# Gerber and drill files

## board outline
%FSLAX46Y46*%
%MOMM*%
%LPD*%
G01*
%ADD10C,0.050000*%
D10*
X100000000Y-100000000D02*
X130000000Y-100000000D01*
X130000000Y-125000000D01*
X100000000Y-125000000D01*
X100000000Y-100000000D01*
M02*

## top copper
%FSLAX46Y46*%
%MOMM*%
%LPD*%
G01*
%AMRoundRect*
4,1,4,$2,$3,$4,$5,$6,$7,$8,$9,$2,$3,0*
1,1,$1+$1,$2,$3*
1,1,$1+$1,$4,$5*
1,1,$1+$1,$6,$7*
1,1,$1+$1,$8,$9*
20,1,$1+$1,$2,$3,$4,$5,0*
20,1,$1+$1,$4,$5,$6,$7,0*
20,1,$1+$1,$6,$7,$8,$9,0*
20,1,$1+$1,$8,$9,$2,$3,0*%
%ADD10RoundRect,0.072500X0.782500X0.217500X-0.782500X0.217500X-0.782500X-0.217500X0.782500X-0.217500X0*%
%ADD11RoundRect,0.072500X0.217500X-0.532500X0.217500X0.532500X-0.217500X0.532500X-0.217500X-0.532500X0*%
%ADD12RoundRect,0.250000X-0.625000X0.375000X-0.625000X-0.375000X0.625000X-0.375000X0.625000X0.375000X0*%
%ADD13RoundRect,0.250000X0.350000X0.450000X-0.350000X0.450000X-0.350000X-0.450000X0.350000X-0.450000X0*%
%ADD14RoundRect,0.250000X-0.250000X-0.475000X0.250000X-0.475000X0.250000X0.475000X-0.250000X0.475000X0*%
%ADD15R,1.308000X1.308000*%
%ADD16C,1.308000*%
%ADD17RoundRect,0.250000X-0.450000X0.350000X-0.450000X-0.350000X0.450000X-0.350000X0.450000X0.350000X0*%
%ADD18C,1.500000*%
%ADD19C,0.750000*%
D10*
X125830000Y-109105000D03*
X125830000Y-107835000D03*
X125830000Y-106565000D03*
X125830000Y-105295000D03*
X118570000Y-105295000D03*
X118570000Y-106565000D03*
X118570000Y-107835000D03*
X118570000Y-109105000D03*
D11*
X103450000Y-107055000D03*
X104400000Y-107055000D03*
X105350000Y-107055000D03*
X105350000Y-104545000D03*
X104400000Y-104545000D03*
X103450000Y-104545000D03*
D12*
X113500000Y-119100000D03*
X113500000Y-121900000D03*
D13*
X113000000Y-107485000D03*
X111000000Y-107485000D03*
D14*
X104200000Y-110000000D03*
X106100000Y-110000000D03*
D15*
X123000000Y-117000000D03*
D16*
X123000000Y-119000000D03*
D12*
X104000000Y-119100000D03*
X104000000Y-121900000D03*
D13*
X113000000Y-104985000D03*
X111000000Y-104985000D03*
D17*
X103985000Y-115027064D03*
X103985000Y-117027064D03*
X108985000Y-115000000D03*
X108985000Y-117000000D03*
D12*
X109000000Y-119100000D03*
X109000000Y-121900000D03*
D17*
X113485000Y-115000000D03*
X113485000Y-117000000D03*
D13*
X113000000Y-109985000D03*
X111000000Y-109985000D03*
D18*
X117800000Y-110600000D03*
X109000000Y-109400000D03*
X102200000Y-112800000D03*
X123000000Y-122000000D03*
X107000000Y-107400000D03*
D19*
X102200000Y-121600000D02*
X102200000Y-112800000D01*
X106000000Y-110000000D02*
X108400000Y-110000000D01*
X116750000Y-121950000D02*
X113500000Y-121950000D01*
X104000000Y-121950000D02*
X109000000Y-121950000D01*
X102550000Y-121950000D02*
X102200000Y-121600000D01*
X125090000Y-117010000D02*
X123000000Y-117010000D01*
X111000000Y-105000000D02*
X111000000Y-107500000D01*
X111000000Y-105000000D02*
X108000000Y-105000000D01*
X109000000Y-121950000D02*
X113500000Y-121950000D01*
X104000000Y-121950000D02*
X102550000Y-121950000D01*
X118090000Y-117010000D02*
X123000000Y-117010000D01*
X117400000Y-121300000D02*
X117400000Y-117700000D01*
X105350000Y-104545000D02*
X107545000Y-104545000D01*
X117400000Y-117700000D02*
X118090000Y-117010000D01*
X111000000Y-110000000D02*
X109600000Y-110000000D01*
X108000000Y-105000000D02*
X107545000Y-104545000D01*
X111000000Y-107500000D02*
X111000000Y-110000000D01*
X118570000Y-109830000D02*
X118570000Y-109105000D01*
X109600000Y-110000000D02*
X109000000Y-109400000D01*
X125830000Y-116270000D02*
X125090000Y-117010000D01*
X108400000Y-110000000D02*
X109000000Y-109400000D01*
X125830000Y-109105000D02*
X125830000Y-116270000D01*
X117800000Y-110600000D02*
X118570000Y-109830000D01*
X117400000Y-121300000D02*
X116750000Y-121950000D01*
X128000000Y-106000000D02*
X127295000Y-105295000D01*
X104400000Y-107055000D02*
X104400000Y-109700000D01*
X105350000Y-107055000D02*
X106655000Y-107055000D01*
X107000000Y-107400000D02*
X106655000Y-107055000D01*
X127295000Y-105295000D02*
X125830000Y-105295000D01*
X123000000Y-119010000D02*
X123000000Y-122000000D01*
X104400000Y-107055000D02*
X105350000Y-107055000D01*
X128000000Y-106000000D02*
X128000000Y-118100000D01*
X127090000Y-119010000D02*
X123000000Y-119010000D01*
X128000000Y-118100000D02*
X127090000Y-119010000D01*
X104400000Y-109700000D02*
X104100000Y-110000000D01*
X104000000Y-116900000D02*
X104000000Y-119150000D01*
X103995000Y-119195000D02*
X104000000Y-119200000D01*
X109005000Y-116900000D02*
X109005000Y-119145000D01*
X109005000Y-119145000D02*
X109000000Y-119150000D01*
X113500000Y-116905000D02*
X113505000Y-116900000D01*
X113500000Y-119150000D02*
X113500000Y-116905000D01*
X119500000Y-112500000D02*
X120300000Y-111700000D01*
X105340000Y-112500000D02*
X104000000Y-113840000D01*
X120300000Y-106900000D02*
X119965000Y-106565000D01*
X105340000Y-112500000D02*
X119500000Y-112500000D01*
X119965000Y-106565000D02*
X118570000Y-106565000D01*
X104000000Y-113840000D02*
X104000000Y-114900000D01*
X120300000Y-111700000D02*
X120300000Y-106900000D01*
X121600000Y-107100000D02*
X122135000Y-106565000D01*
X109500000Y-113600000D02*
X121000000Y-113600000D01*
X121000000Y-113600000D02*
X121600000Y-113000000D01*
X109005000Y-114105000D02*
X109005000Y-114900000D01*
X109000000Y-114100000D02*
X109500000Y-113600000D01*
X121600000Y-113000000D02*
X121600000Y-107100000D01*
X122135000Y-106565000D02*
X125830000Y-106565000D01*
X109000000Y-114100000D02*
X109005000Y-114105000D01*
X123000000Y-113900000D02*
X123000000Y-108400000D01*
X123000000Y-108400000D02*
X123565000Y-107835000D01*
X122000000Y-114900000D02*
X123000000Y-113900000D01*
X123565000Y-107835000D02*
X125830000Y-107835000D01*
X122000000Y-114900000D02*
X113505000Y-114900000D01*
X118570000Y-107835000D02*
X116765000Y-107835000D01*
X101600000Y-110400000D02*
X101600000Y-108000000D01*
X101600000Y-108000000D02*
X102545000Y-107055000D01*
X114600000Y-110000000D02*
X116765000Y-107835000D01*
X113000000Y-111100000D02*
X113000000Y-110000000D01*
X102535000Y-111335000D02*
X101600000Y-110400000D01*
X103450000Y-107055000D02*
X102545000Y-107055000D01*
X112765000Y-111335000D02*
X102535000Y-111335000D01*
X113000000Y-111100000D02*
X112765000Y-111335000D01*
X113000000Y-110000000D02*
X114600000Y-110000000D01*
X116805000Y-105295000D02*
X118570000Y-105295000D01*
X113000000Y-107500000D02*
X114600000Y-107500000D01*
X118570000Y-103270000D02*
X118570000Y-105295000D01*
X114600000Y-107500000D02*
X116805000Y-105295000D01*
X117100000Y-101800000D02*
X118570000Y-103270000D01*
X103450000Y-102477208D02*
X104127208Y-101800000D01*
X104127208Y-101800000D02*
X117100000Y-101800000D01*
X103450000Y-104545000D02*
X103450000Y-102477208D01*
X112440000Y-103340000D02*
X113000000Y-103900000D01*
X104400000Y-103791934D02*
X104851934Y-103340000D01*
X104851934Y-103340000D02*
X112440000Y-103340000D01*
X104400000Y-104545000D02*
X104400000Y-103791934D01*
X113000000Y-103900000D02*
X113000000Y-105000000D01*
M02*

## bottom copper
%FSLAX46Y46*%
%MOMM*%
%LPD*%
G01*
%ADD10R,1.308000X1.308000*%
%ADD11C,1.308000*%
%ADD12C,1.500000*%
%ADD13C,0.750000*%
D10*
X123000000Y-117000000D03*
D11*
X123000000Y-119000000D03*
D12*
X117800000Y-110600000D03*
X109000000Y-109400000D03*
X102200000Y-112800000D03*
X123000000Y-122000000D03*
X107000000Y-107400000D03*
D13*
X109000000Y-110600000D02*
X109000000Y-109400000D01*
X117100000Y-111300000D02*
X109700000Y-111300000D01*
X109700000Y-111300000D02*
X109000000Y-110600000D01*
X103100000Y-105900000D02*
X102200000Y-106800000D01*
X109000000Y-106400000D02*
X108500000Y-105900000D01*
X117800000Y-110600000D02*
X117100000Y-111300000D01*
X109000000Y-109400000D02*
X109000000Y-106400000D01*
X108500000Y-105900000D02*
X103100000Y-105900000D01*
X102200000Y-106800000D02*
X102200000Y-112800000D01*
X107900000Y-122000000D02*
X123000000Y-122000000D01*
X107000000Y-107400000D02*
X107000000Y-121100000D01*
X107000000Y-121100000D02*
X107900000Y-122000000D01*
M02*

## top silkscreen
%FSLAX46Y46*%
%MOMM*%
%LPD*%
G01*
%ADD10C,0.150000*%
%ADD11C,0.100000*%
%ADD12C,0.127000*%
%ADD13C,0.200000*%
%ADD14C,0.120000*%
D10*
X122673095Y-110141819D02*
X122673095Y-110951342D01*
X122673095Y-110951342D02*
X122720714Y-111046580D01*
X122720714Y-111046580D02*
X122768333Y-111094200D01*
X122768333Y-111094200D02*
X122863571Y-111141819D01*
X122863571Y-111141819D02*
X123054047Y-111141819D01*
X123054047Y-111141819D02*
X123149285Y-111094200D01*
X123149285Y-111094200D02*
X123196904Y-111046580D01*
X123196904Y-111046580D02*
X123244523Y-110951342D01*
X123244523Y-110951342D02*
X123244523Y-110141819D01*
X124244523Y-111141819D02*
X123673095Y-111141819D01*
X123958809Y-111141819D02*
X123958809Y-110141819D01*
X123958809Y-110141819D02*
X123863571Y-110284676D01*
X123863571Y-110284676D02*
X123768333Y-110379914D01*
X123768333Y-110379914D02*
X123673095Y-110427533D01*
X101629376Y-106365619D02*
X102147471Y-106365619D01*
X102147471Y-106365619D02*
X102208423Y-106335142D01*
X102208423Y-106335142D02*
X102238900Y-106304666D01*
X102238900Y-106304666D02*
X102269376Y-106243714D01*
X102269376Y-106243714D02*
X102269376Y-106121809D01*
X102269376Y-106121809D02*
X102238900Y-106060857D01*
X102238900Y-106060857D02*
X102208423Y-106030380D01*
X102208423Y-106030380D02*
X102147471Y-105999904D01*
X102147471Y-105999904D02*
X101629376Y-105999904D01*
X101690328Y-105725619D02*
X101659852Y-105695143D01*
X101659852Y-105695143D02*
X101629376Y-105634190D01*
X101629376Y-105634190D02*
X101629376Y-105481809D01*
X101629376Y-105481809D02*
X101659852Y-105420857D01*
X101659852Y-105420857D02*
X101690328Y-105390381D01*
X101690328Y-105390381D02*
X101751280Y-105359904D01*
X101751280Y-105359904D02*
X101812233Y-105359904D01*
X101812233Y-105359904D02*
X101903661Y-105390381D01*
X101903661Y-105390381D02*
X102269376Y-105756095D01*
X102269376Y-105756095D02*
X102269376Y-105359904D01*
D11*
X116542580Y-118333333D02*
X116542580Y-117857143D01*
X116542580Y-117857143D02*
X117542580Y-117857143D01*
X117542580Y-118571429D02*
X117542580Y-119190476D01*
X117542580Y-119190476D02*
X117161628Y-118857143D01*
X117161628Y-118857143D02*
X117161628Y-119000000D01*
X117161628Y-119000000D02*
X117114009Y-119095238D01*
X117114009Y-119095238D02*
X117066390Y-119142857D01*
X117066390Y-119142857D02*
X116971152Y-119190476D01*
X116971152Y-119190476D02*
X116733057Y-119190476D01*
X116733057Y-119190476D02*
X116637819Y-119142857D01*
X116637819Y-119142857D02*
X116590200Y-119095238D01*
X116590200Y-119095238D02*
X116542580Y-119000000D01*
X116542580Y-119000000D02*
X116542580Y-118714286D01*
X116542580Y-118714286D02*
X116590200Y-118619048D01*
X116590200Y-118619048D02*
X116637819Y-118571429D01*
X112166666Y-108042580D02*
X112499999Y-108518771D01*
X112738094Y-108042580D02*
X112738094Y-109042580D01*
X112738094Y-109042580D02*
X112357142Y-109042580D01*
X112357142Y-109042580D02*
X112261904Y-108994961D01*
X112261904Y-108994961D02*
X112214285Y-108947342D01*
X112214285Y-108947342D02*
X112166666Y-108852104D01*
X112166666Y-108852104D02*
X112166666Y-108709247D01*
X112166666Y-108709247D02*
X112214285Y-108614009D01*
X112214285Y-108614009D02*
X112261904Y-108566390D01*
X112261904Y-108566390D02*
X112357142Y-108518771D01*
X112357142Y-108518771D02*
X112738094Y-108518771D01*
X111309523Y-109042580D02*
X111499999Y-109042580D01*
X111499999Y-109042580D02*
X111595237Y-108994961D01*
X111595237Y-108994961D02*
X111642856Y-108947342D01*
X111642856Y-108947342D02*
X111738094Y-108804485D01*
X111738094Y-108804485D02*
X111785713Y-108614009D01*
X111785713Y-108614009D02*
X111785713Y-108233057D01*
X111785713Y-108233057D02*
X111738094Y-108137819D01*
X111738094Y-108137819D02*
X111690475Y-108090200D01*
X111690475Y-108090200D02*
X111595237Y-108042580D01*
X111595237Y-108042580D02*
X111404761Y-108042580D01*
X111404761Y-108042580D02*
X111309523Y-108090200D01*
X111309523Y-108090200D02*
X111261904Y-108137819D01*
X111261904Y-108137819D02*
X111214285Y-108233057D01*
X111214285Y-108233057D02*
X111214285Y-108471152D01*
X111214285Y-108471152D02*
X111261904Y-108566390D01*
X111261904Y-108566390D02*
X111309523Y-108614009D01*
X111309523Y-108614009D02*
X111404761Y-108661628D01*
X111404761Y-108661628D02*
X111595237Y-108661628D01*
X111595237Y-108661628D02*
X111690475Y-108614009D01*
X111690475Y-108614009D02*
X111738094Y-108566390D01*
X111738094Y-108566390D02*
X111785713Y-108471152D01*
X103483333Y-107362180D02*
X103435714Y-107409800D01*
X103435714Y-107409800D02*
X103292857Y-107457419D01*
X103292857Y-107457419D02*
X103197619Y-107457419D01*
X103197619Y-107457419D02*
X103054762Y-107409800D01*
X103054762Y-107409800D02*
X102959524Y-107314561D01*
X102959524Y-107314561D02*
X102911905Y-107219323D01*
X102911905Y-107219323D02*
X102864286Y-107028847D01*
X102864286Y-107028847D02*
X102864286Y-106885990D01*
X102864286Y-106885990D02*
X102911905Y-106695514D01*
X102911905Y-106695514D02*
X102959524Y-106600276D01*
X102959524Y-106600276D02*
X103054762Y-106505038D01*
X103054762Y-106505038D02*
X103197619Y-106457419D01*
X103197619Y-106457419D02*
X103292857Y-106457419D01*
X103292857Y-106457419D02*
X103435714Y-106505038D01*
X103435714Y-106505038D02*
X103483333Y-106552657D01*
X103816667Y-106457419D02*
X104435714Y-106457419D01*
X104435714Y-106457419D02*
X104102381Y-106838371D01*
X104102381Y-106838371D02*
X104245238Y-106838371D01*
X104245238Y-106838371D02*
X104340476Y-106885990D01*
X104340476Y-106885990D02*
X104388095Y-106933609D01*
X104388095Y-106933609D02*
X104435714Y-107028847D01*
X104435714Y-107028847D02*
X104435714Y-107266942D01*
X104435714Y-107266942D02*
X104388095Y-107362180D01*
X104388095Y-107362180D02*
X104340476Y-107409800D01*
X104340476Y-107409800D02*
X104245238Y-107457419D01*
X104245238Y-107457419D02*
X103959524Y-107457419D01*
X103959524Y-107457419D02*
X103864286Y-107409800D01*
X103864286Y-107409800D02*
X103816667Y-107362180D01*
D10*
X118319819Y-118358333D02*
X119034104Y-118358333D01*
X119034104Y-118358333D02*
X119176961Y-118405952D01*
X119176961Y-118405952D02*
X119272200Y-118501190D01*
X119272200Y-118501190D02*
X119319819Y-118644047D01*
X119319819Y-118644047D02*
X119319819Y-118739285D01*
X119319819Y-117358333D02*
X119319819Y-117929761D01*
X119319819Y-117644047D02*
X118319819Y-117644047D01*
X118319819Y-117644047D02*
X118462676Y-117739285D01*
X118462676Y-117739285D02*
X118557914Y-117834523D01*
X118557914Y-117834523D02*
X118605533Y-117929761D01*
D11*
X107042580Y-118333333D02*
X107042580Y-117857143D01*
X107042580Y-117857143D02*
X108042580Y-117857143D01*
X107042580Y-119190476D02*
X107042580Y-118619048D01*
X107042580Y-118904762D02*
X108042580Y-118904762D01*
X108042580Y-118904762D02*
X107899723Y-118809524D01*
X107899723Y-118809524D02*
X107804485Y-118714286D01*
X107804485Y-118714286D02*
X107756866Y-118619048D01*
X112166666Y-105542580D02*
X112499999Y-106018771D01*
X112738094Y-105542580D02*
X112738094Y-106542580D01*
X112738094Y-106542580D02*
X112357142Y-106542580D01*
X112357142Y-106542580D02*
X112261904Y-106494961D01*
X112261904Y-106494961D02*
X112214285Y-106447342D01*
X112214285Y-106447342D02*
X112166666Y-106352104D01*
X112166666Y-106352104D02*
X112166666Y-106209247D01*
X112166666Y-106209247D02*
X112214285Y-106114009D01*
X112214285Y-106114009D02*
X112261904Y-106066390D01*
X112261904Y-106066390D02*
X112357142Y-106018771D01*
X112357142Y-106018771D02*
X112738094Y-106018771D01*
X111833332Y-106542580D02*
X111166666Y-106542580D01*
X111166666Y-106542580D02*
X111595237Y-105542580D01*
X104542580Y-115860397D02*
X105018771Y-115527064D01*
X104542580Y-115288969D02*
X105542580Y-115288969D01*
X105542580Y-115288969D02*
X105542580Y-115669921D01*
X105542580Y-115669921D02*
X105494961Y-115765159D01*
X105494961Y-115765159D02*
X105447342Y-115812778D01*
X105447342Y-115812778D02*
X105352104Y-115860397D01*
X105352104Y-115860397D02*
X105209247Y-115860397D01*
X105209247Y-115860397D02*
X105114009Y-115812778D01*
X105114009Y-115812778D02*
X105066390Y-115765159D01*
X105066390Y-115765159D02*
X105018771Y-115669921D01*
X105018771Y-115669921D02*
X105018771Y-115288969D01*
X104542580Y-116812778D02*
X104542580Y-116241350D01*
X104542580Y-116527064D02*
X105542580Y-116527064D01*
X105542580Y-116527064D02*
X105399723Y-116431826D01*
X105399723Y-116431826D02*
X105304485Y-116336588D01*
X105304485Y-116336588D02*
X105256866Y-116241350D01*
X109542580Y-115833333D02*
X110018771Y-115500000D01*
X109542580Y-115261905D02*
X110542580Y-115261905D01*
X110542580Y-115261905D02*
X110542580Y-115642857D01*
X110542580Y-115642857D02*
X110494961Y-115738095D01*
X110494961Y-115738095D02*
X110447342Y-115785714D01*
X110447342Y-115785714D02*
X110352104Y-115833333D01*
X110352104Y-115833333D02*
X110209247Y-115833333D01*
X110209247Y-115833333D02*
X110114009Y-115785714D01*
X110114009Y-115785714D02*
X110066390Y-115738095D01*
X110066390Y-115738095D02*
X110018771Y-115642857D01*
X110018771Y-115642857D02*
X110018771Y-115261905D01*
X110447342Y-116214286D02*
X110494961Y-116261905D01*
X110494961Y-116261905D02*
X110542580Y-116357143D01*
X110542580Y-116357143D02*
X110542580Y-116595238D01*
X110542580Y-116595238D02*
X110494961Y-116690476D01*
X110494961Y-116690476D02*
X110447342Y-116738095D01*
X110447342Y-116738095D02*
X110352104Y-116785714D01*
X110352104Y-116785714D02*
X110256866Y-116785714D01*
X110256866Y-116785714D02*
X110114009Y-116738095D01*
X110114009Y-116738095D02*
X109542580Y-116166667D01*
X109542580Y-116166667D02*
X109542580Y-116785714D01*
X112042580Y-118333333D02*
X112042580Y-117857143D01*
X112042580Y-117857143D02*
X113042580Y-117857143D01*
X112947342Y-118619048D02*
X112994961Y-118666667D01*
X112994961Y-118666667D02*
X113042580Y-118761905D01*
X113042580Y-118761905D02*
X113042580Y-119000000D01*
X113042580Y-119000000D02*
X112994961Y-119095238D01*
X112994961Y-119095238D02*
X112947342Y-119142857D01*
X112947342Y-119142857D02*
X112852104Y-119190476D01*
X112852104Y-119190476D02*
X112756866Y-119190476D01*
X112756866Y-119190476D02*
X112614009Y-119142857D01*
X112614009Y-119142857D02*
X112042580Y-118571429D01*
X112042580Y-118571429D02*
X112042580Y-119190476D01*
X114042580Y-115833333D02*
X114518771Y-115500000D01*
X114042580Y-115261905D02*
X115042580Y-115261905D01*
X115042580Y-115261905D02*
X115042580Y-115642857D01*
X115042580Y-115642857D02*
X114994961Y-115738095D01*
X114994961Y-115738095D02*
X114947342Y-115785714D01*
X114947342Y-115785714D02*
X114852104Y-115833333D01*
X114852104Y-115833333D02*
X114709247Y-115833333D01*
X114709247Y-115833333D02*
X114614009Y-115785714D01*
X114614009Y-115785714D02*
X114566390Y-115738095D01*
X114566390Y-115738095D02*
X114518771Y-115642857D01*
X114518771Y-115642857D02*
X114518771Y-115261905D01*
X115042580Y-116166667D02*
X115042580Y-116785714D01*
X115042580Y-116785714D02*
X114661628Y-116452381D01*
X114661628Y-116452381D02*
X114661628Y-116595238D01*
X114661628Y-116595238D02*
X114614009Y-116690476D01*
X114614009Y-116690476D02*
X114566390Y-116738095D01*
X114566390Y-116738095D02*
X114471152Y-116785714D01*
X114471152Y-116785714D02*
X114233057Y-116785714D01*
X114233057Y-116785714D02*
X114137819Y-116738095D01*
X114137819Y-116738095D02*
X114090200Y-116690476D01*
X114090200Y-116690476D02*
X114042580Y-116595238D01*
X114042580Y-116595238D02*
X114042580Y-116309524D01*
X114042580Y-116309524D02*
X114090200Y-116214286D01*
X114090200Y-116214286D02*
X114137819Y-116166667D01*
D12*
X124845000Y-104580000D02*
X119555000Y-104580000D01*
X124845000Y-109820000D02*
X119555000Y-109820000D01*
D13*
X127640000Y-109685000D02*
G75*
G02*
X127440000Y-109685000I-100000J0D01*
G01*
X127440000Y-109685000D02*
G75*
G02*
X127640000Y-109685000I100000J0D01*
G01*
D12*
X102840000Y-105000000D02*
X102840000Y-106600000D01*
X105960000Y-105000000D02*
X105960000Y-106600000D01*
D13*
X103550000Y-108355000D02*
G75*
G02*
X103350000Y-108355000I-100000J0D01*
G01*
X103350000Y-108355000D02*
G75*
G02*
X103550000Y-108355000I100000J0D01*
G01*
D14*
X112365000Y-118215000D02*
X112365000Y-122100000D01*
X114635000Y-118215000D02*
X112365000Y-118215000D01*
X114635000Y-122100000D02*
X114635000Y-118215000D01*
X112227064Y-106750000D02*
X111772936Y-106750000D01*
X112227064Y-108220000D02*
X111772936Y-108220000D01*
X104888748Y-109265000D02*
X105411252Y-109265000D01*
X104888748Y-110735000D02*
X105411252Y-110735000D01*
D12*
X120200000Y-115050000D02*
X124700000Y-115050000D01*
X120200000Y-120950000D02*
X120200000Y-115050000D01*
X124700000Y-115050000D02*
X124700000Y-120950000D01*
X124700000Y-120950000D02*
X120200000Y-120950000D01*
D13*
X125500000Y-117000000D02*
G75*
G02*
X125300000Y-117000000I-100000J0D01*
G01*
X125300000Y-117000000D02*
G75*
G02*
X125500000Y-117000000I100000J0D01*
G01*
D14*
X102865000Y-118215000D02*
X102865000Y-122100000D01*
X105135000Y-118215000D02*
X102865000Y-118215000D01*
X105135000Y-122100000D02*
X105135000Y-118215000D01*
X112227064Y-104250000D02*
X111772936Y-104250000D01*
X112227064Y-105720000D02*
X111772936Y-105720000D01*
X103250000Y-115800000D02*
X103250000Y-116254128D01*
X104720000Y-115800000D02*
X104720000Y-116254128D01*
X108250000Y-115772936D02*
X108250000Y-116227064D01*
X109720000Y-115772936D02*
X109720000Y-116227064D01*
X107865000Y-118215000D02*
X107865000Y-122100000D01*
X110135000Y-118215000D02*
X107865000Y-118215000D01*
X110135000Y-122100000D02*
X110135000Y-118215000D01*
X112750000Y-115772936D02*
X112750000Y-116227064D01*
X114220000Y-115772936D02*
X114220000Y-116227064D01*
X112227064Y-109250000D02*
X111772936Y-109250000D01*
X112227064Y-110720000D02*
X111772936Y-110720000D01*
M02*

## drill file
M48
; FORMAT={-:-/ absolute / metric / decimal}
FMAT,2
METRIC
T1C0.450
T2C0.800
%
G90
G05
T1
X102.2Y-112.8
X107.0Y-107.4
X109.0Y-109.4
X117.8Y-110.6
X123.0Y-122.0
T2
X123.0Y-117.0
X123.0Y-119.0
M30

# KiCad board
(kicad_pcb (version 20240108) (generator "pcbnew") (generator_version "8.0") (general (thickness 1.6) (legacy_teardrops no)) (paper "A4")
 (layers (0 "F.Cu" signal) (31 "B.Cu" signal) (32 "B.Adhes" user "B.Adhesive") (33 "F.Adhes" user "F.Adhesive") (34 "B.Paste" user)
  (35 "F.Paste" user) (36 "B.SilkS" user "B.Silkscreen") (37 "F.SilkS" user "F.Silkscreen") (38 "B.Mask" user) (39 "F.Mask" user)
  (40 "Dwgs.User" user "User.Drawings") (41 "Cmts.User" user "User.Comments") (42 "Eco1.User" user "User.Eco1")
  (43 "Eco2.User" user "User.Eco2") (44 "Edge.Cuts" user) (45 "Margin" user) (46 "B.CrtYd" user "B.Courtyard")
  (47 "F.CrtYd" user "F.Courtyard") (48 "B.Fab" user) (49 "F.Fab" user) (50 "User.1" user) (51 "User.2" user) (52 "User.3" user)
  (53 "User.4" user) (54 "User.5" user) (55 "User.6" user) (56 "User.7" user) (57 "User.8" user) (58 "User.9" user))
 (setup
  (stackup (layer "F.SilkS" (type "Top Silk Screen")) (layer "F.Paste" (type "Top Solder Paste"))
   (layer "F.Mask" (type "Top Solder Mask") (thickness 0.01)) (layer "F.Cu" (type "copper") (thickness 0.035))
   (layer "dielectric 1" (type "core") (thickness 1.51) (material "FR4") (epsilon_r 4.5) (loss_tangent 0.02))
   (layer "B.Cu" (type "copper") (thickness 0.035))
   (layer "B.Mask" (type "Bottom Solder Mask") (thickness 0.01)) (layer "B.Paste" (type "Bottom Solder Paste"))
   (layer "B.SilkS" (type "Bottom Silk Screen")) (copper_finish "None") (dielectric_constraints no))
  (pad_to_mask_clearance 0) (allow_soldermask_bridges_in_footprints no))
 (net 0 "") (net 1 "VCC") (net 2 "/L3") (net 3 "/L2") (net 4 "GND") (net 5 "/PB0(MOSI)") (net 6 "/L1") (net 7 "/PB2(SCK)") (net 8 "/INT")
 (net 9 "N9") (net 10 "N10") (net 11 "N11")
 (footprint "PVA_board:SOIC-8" (layer "F.Cu") (at 122.2 107.2 180)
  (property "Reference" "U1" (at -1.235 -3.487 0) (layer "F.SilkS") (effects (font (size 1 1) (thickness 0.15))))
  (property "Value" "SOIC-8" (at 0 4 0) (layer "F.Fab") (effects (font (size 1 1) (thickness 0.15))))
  (fp_line (start -2.645 2.62) (end 2.645 2.62) (stroke (width 0.127) (type solid)) (layer "F.SilkS"))
  (fp_line (start -2.645 -2.62) (end 2.645 -2.62) (stroke (width 0.127) (type solid)) (layer "F.SilkS"))
  (fp_circle (center -5.34 -2.485) (end -5.24 -2.485) (stroke (width 0.2) (type solid)) (fill none) (layer "F.SilkS"))
  (pad "1" smd roundrect (at -3.63 -1.905 180) (size 1.71 0.58) (layers "F.Cu" "F.Paste" "F.Mask") (roundrect_rratio 0.125) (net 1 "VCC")
   (solder_mask_margin 0.102))
  (pad "2" smd roundrect (at -3.63 -0.635 180) (size 1.71 0.58) (layers "F.Cu" "F.Paste" "F.Mask") (roundrect_rratio 0.125) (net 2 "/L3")
   (solder_mask_margin 0.102))
  (pad "3" smd roundrect (at -3.63 0.635 180) (size 1.71 0.58) (layers "F.Cu" "F.Paste" "F.Mask") (roundrect_rratio 0.125) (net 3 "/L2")
   (solder_mask_margin 0.102))
  (pad "4" smd roundrect (at -3.63 1.905 180) (size 1.71 0.58) (layers "F.Cu" "F.Paste" "F.Mask") (roundrect_rratio 0.125) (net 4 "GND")
   (solder_mask_margin 0.102))
  (pad "5" smd roundrect (at 3.63 1.905 180) (size 1.71 0.58) (layers "F.Cu" "F.Paste" "F.Mask") (roundrect_rratio 0.125)
   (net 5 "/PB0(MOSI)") (solder_mask_margin 0.102))
  (pad "6" smd roundrect (at 3.63 0.635 180) (size 1.71 0.58) (layers "F.Cu" "F.Paste" "F.Mask") (roundrect_rratio 0.125) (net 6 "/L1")
   (solder_mask_margin 0.102))
  (pad "7" smd roundrect (at 3.63 -0.635 180) (size 1.71 0.58) (layers "F.Cu" "F.Paste" "F.Mask") (roundrect_rratio 0.125)
   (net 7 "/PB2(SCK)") (solder_mask_margin 0.102))
  (pad "8" smd roundrect (at 3.63 -1.905 180) (size 1.71 0.58) (layers "F.Cu" "F.Paste" "F.Mask") (roundrect_rratio 0.125) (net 1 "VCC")
   (solder_mask_margin 0.102)))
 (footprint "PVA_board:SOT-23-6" (layer "F.Cu") (at 104.4 105.8 90)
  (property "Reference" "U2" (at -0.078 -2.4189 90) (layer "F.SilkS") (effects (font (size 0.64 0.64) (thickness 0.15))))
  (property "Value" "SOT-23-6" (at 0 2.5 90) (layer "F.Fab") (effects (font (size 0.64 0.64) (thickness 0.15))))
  (fp_line (start 0.8 -1.56) (end -0.8 -1.56) (stroke (width 0.127) (type solid)) (layer "F.SilkS"))
  (fp_line (start 0.8 1.56) (end -0.8 1.56) (stroke (width 0.127) (type solid)) (layer "F.SilkS"))
  (fp_circle (center -2.555 -0.95) (end -2.455 -0.95) (stroke (width 0.2) (type solid)) (fill none) (layer "F.SilkS"))
  (pad "1" smd roundrect (at -1.255 -0.95 90) (size 1.21 0.58) (layers "F.Cu" "F.Paste" "F.Mask") (roundrect_rratio 0.125)
   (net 7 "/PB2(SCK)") (solder_mask_margin 0.102))
  (pad "2" smd roundrect (at -1.255 0 90) (size 1.21 0.58) (layers "F.Cu" "F.Paste" "F.Mask") (roundrect_rratio 0.125) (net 4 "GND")
   (solder_mask_margin 0.102))
  (pad "3" smd roundrect (at -1.255 0.95 90) (size 1.21 0.58) (layers "F.Cu" "F.Paste" "F.Mask") (roundrect_rratio 0.125) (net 4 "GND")
   (solder_mask_margin 0.102))
  (pad "4" smd roundrect (at 1.255 0.95 90) (size 1.21 0.58) (layers "F.Cu" "F.Paste" "F.Mask") (roundrect_rratio 0.125) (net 1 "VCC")
   (solder_mask_margin 0.102))
  (pad "5" smd roundrect (at 1.255 0 90) (size 1.21 0.58) (layers "F.Cu" "F.Paste" "F.Mask") (roundrect_rratio 0.125) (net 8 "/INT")
   (solder_mask_margin 0.102))
  (pad "6" smd roundrect (at 1.255 -0.95 90) (size 1.21 0.58) (layers "F.Cu" "F.Paste" "F.Mask") (roundrect_rratio 0.125)
   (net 5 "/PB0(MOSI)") (solder_mask_margin 0.102)))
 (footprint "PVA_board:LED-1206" (layer "F.Cu") (at 113.5 120.5 -90)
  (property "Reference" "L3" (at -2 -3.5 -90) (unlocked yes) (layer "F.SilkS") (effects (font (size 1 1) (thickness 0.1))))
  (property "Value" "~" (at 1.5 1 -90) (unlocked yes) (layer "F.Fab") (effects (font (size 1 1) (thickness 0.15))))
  (fp_line (start -2.285 1.135) (end 1.6 1.135) (stroke (width 0.12) (type solid)) (layer "F.SilkS"))
  (fp_line (start -2.285 -1.135) (end -2.285 1.135) (stroke (width 0.12) (type solid)) (layer "F.SilkS"))
  (fp_line (start 1.6 -1.135) (end -2.285 -1.135) (stroke (width 0.12) (type solid)) (layer "F.SilkS"))
  (pad "1" smd roundrect (at -1.4 0 270) (size 1.25 1.75) (layers "F.Cu" "F.Paste" "F.Mask") (roundrect_rratio 0.2) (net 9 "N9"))
  (pad "2" smd roundrect (at 1.4 0 270) (size 1.25 1.75) (layers "F.Cu" "F.Paste" "F.Mask") (roundrect_rratio 0.2) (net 1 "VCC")))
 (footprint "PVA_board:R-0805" (layer "F.Cu") (at 112 107.5 180)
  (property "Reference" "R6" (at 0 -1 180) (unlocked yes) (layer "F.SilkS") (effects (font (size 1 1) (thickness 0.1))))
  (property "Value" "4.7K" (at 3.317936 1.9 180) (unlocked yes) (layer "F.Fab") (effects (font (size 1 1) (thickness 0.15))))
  (fp_line (start -0.227064 0.75) (end 0.227064 0.75) (stroke (width 0.12) (type solid)) (layer "F.SilkS"))
  (fp_line (start -0.227064 -0.72) (end 0.227064 -0.72) (stroke (width 0.12) (type solid)) (layer "F.SilkS"))
  (pad "1" smd roundrect (at -1 0.015 180) (size 1.2 1.4) (layers "F.Cu" "F.Paste" "F.Mask") (roundrect_rratio 0.208333)
   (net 5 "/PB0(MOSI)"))
  (pad "2" smd roundrect (at 1 0.015 180) (size 1.2 1.4) (layers "F.Cu" "F.Paste" "F.Mask") (roundrect_rratio 0.208333) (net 1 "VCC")))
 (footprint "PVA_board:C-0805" (layer "F.Cu") (at 105.15 110)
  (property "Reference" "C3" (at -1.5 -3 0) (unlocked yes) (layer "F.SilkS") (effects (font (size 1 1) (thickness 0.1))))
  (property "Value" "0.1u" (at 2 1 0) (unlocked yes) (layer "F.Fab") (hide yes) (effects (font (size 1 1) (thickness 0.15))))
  (fp_line (start -0.261252 -0.735) (end 0.261252 -0.735) (stroke (width 0.12) (type solid)) (layer "F.SilkS"))
  (fp_line (start -0.261252 0.735) (end 0.261252 0.735) (stroke (width 0.12) (type solid)) (layer "F.SilkS"))
  (pad "1" smd roundrect (at -0.95 0) (size 1 1.45) (layers "F.Cu" "F.Paste" "F.Mask") (roundrect_rratio 0.25) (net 4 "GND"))
  (pad "2" smd roundrect (at 0.95 0) (size 1 1.45) (layers "F.Cu" "F.Paste" "F.Mask") (roundrect_rratio 0.25) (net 1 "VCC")))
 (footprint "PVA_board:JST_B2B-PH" (layer "F.Cu") (at 123 118 90)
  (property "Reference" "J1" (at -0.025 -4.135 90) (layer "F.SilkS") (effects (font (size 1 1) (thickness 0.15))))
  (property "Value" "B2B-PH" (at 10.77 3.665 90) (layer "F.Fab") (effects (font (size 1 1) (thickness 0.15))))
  (fp_line (start 2.95 -2.8) (end 2.95 1.7) (stroke (width 0.127) (type solid)) (layer "F.SilkS"))
  (fp_line (start -2.95 -2.8) (end 2.95 -2.8) (stroke (width 0.127) (type solid)) (layer "F.SilkS"))
  (fp_line (start 2.95 1.7) (end -2.95 1.7) (stroke (width 0.127) (type solid)) (layer "F.SilkS"))
  (fp_line (start -2.95 1.7) (end -2.95 -2.8) (stroke (width 0.127) (type solid)) (layer "F.SilkS"))
  (fp_circle (center 1 2.4) (end 1.1 2.4) (stroke (width 0.2) (type solid)) (fill none) (layer "F.SilkS"))
  (pad "1" thru_hole rect (at 1 0 90) (size 1.308 1.308) (drill 0.8) (layers "*.Cu" "*.Mask") (remove_unused_layers no) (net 1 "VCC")
   (solder_mask_margin 0.102))
  (pad "2" thru_hole circle (at -1 0 90) (size 1.308 1.308) (drill 0.8) (layers "*.Cu" "*.Mask") (remove_unused_layers no) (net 4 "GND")
   (solder_mask_margin 0.102)))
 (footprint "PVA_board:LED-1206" (layer "F.Cu") (at 104 120.5 -90)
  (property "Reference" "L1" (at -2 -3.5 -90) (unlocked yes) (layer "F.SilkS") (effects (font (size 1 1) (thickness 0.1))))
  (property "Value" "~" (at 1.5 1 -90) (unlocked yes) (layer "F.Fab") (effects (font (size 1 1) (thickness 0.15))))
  (fp_line (start -2.285 1.135) (end 1.6 1.135) (stroke (width 0.12) (type solid)) (layer "F.SilkS"))
  (fp_line (start -2.285 -1.135) (end -2.285 1.135) (stroke (width 0.12) (type solid)) (layer "F.SilkS"))
  (fp_line (start 1.6 -1.135) (end -2.285 -1.135) (stroke (width 0.12) (type solid)) (layer "F.SilkS"))
  (pad "1" smd roundrect (at -1.4 0 270) (size 1.25 1.75) (layers "F.Cu" "F.Paste" "F.Mask") (roundrect_rratio 0.2) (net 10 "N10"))
  (pad "2" smd roundrect (at 1.4 0 270) (size 1.25 1.75) (layers "F.Cu" "F.Paste" "F.Mask") (roundrect_rratio 0.2) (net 1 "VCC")))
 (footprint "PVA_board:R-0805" (layer "F.Cu") (at 112 105 180)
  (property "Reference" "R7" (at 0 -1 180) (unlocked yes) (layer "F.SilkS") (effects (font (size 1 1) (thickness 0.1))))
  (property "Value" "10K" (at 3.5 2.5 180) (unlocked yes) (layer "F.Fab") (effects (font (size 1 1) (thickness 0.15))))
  (fp_line (start -0.227064 0.75) (end 0.227064 0.75) (stroke (width 0.12) (type solid)) (layer "F.SilkS"))
  (fp_line (start -0.227064 -0.72) (end 0.227064 -0.72) (stroke (width 0.12) (type solid)) (layer "F.SilkS"))
  (pad "1" smd roundrect (at -1 0.015 180) (size 1.2 1.4) (layers "F.Cu" "F.Paste" "F.Mask") (roundrect_rratio 0.208333) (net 8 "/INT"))
  (pad "2" smd roundrect (at 1 0.015 180) (size 1.2 1.4) (layers "F.Cu" "F.Paste" "F.Mask") (roundrect_rratio 0.208333) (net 1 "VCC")))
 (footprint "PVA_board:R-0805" (layer "F.Cu") (at 104 116.027064 -90)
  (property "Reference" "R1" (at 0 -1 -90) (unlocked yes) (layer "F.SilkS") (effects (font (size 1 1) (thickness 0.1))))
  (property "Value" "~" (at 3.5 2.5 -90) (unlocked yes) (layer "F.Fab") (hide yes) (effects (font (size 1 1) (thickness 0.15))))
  (fp_line (start -0.227064 0.75) (end 0.227064 0.75) (stroke (width 0.12) (type solid)) (layer "F.SilkS"))
  (fp_line (start -0.227064 -0.72) (end 0.227064 -0.72) (stroke (width 0.12) (type solid)) (layer "F.SilkS"))
  (pad "1" smd roundrect (at -1 0.015 270) (size 1.2 1.4) (layers "F.Cu" "F.Paste" "F.Mask") (roundrect_rratio 0.208333) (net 6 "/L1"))
  (pad "2" smd roundrect (at 1 0.015 270) (size 1.2 1.4) (layers "F.Cu" "F.Paste" "F.Mask") (roundrect_rratio 0.208333) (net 10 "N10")))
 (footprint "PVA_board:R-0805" (layer "F.Cu") (at 109 116 -90)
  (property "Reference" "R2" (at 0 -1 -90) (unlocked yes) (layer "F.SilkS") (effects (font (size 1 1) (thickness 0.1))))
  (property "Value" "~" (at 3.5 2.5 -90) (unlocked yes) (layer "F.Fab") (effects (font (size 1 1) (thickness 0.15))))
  (fp_line (start -0.227064 0.75) (end 0.227064 0.75) (stroke (width 0.12) (type solid)) (layer "F.SilkS"))
  (fp_line (start -0.227064 -0.72) (end 0.227064 -0.72) (stroke (width 0.12) (type solid)) (layer "F.SilkS"))
  (pad "1" smd roundrect (at -1 0.015 270) (size 1.2 1.4) (layers "F.Cu" "F.Paste" "F.Mask") (roundrect_rratio 0.208333) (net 3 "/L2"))
  (pad "2" smd roundrect (at 1 0.015 270) (size 1.2 1.4) (layers "F.Cu" "F.Paste" "F.Mask") (roundrect_rratio 0.208333) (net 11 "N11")))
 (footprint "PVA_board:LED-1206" (layer "F.Cu") (at 109 120.5 -90)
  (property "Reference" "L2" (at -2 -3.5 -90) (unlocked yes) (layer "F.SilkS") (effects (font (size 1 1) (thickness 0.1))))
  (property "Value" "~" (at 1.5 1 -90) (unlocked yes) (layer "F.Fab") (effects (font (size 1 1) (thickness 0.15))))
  (fp_line (start -2.285 1.135) (end 1.6 1.135) (stroke (width 0.12) (type solid)) (layer "F.SilkS"))
  (fp_line (start -2.285 -1.135) (end -2.285 1.135) (stroke (width 0.12) (type solid)) (layer "F.SilkS"))
  (fp_line (start 1.6 -1.135) (end -2.285 -1.135) (stroke (width 0.12) (type solid)) (layer "F.SilkS"))
  (pad "1" smd roundrect (at -1.4 0 270) (size 1.25 1.75) (layers "F.Cu" "F.Paste" "F.Mask") (roundrect_rratio 0.2) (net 11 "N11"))
  (pad "2" smd roundrect (at 1.4 0 270) (size 1.25 1.75) (layers "F.Cu" "F.Paste" "F.Mask") (roundrect_rratio 0.2) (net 1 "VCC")))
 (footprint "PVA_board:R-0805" (layer "F.Cu") (at 113.5 116 -90)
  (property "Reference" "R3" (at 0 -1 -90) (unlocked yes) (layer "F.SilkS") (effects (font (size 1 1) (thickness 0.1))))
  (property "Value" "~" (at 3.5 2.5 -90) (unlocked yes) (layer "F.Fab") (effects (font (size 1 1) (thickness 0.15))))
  (fp_line (start -0.227064 0.75) (end 0.227064 0.75) (stroke (width 0.12) (type solid)) (layer "F.SilkS"))
  (fp_line (start -0.227064 -0.72) (end 0.227064 -0.72) (stroke (width 0.12) (type solid)) (layer "F.SilkS"))
  (pad "1" smd roundrect (at -1 0.015 270) (size 1.2 1.4) (layers "F.Cu" "F.Paste" "F.Mask") (roundrect_rratio 0.208333) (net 2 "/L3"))
  (pad "2" smd roundrect (at 1 0.015 270) (size 1.2 1.4) (layers "F.Cu" "F.Paste" "F.Mask") (roundrect_rratio 0.208333) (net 9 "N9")))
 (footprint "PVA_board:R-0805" (layer "F.Cu") (at 112 110 180)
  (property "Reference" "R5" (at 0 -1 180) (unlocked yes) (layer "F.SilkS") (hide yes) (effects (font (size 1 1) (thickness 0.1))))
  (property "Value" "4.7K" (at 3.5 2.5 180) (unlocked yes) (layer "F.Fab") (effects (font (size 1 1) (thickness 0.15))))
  (fp_line (start -0.227064 0.75) (end 0.227064 0.75) (stroke (width 0.12) (type solid)) (layer "F.SilkS"))
  (fp_line (start -0.227064 -0.72) (end 0.227064 -0.72) (stroke (width 0.12) (type solid)) (layer "F.SilkS"))
  (pad "1" smd roundrect (at -1 0.015 180) (size 1.2 1.4) (layers "F.Cu" "F.Paste" "F.Mask") (roundrect_rratio 0.208333) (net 7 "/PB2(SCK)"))
  (pad "2" smd roundrect (at 1 0.015 180) (size 1.2 1.4) (layers "F.Cu" "F.Paste" "F.Mask") (roundrect_rratio 0.208333) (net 1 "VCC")))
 (gr_rect (start 100 100) (end 130 125) (stroke (width 0.05) (type default)) (fill none) (layer "Edge.Cuts"))
 (segment (start 102.2 121.6) (end 102.2 112.8) (width 0.75) (layer "F.Cu") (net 1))
 (segment (start 106 110) (end 108.4 110) (width 0.75) (layer "F.Cu") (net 1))
 (segment (start 116.75 121.95) (end 113.5 121.95) (width 0.75) (layer "F.Cu") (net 1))
 (segment (start 104 121.95) (end 109 121.95) (width 0.75) (layer "F.Cu") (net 1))
 (segment (start 102.55 121.95) (end 102.2 121.6) (width 0.75) (layer "F.Cu") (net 1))
 (segment (start 125.09 117.01) (end 123 117.01) (width 0.75) (layer "F.Cu") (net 1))
 (segment (start 111 105) (end 111 107.5) (width 0.75) (layer "F.Cu") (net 1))
 (segment (start 111 105) (end 108 105) (width 0.75) (layer "F.Cu") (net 1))
 (segment (start 109 121.95) (end 113.5 121.95) (width 0.75) (layer "F.Cu") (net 1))
 (segment (start 104 121.95) (end 102.55 121.95) (width 0.75) (layer "F.Cu") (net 1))
 (segment (start 118.09 117.01) (end 123 117.01) (width 0.75) (layer "F.Cu") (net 1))
 (segment (start 117.4 121.3) (end 117.4 117.7) (width 0.75) (layer "F.Cu") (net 1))
 (segment (start 105.35 104.545) (end 107.545 104.545) (width 0.75) (layer "F.Cu") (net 1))
 (segment (start 117.4 117.7) (end 118.09 117.01) (width 0.75) (layer "F.Cu") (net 1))
 (segment (start 111 110) (end 109.6 110) (width 0.75) (layer "F.Cu") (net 1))
 (segment (start 108 105) (end 107.545 104.545) (width 0.75) (layer "F.Cu") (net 1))
 (segment (start 111 107.5) (end 111 110) (width 0.75) (layer "F.Cu") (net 1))
 (segment (start 118.57 109.83) (end 118.57 109.105) (width 0.75) (layer "F.Cu") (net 1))
 (segment (start 109.6 110) (end 109 109.4) (width 0.75) (layer "F.Cu") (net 1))
 (segment (start 125.83 116.27) (end 125.09 117.01) (width 0.75) (layer "F.Cu") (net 1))
 (segment (start 108.4 110) (end 109 109.4) (width 0.75) (layer "F.Cu") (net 1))
 (segment (start 125.83 109.105) (end 125.83 116.27) (width 0.75) (layer "F.Cu") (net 1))
 (segment (start 117.8 110.6) (end 118.57 109.83) (width 0.75) (layer "F.Cu") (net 1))
 (segment (start 117.4 121.3) (end 116.75 121.95) (width 0.75) (layer "F.Cu") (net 1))
 (via (at 117.8 110.6) (size 1.5) (drill 0.45) (layers "F.Cu" "B.Cu") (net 1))
 (via (at 109 109.4) (size 1.5) (drill 0.45) (layers "F.Cu" "B.Cu") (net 1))
 (via (at 102.2 112.8) (size 1.5) (drill 0.45) (layers "F.Cu" "B.Cu") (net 1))
 (segment (start 109 110.6) (end 109 109.4) (width 0.75) (layer "B.Cu") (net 1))
 (segment (start 117.1 111.3) (end 109.7 111.3) (width 0.75) (layer "B.Cu") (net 1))
 (segment (start 109.7 111.3) (end 109 110.6) (width 0.75) (layer "B.Cu") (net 1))
 (segment (start 103.1 105.9) (end 102.2 106.8) (width 0.75) (layer "B.Cu") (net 1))
 (segment (start 109 106.4) (end 108.5 105.9) (width 0.75) (layer "B.Cu") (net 1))
 (segment (start 117.8 110.6) (end 117.1 111.3) (width 0.75) (layer "B.Cu") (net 1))
 (segment (start 109 109.4) (end 109 106.4) (width 0.75) (layer "B.Cu") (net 1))
 (segment (start 108.5 105.9) (end 103.1 105.9) (width 0.75) (layer "B.Cu") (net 1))
 (segment (start 102.2 106.8) (end 102.2 112.8) (width 0.75) (layer "B.Cu") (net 1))
 (segment (start 128 106) (end 127.295 105.295) (width 0.75) (layer "F.Cu") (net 4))
 (segment (start 104.4 107.055) (end 104.4 109.7) (width 0.75) (layer "F.Cu") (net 4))
 (segment (start 105.35 107.055) (end 106.655 107.055) (width 0.75) (layer "F.Cu") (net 4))
 (segment (start 107 107.4) (end 106.655 107.055) (width 0.75) (layer "F.Cu") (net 4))
 (segment (start 127.295 105.295) (end 125.83 105.295) (width 0.75) (layer "F.Cu") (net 4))
 (segment (start 123 119.01) (end 123 122) (width 0.75) (layer "F.Cu") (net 4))
 (segment (start 104.4 107.055) (end 105.35 107.055) (width 0.75) (layer "F.Cu") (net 4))
 (segment (start 128 106) (end 128 118.1) (width 0.75) (layer "F.Cu") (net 4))
 (segment (start 127.09 119.01) (end 123 119.01) (width 0.75) (layer "F.Cu") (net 4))
 (segment (start 128 118.1) (end 127.09 119.01) (width 0.75) (layer "F.Cu") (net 4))
 (segment (start 104.4 109.7) (end 104.1 110) (width 0.75) (layer "F.Cu") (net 4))
 (via (at 123 122) (size 1.5) (drill 0.45) (layers "F.Cu" "B.Cu") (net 4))
 (via (at 107 107.4) (size 1.5) (drill 0.45) (layers "F.Cu" "B.Cu") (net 4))
 (segment (start 107.9 122) (end 123 122) (width 0.75) (layer "B.Cu") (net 4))
 (segment (start 107 107.4) (end 107 121.1) (width 0.75) (layer "B.Cu") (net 4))
 (segment (start 107 121.1) (end 107.9 122) (width 0.75) (layer "B.Cu") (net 4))
 (segment (start 104 116.9) (end 104 119.15) (width 0.75) (layer "F.Cu") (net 10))
 (segment (start 103.995 119.195) (end 104 119.2) (width 0.75) (layer "F.Cu") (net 10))
 (segment (start 109.005 116.9) (end 109.005 119.145) (width 0.75) (layer "F.Cu") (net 11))
 (segment (start 109.005 119.145) (end 109 119.15) (width 0.75) (layer "F.Cu") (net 11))
 (segment (start 113.5 116.905) (end 113.505 116.9) (width 0.75) (layer "F.Cu") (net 9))
 (segment (start 113.5 119.15) (end 113.5 116.905) (width 0.75) (layer "F.Cu") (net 9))
 (segment (start 119.5 112.5) (end 120.3 111.7) (width 0.75) (layer "F.Cu") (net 6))
 (segment (start 105.34 112.5) (end 104 113.84) (width 0.75) (layer "F.Cu") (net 6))
 (segment (start 120.3 106.9) (end 119.965 106.565) (width 0.75) (layer "F.Cu") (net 6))
 (segment (start 105.34 112.5) (end 119.5 112.5) (width 0.75) (layer "F.Cu") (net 6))
 (segment (start 119.965 106.565) (end 118.57 106.565) (width 0.75) (layer "F.Cu") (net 6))
 (segment (start 104 113.84) (end 104 114.9) (width 0.75) (layer "F.Cu") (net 6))
 (segment (start 120.3 111.7) (end 120.3 106.9) (width 0.75) (layer "F.Cu") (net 6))
 (segment (start 121.6 107.1) (end 122.135 106.565) (width 0.75) (layer "F.Cu") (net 3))
 (segment (start 109.5 113.6) (end 121 113.6) (width 0.75) (layer "F.Cu") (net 3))
 (segment (start 121 113.6) (end 121.6 113) (width 0.75) (layer "F.Cu") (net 3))
 (segment (start 109.005 114.105) (end 109.005 114.9) (width 0.75) (layer "F.Cu") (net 3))
 (segment (start 109 114.1) (end 109.5 113.6) (width 0.75) (layer "F.Cu") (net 3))
 (segment (start 121.6 113) (end 121.6 107.1) (width 0.75) (layer "F.Cu") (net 3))
 (segment (start 122.135 106.565) (end 125.83 106.565) (width 0.75) (layer "F.Cu") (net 3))
 (segment (start 109 114.1) (end 109.005 114.105) (width 0.75) (layer "F.Cu") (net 3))
 (segment (start 123 113.9) (end 123 108.4) (width 0.75) (layer "F.Cu") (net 2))
 (segment (start 123 108.4) (end 123.565 107.835) (width 0.75) (layer "F.Cu") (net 2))
 (segment (start 122 114.9) (end 123 113.9) (width 0.75) (layer "F.Cu") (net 2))
 (segment (start 123.565 107.835) (end 125.83 107.835) (width 0.75) (layer "F.Cu") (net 2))
 (segment (start 122 114.9) (end 113.505 114.9) (width 0.75) (layer "F.Cu") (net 2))
 (segment (start 118.57 107.835) (end 116.765 107.835) (width 0.75) (layer "F.Cu") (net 7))
 (segment (start 101.6 110.4) (end 101.6 108) (width 0.75) (layer "F.Cu") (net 7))
 (segment (start 101.6 108) (end 102.545 107.055) (width 0.75) (layer "F.Cu") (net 7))
 (segment (start 114.6 110) (end 116.765 107.835) (width 0.75) (layer "F.Cu") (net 7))
 (segment (start 113 111.1) (end 113 110) (width 0.75) (layer "F.Cu") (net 7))
 (segment (start 102.535 111.335) (end 101.6 110.4) (width 0.75) (layer "F.Cu") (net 7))
 (segment (start 103.45 107.055) (end 102.545 107.055) (width 0.75) (layer "F.Cu") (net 7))
 (segment (start 112.765 111.335) (end 102.535 111.335) (width 0.75) (layer "F.Cu") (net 7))
 (segment (start 113 111.1) (end 112.765 111.335) (width 0.75) (layer "F.Cu") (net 7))
 (segment (start 113 110) (end 114.6 110) (width 0.75) (layer "F.Cu") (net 7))
 (segment (start 116.805 105.295) (end 118.57 105.295) (width 0.75) (layer "F.Cu") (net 5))
 (segment (start 113 107.5) (end 114.6 107.5) (width 0.75) (layer "F.Cu") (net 5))
 (segment (start 118.57 103.27) (end 118.57 105.295) (width 0.75) (layer "F.Cu") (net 5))
 (segment (start 114.6 107.5) (end 116.805 105.295) (width 0.75) (layer "F.Cu") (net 5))
 (segment (start 117.1 101.8) (end 118.57 103.27) (width 0.75) (layer "F.Cu") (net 5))
 (segment (start 103.45 102.477208) (end 104.127208 101.8) (width 0.75) (layer "F.Cu") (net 5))
 (segment (start 104.127208 101.8) (end 117.1 101.8) (width 0.75) (layer "F.Cu") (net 5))
 (segment (start 103.45 104.545) (end 103.45 102.477208) (width 0.75) (layer "F.Cu") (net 5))
 (segment (start 112.44 103.34) (end 113 103.9) (width 0.75) (layer "F.Cu") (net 8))
 (segment (start 104.4 103.791934) (end 104.851934 103.34) (width 0.75) (layer "F.Cu") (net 8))
 (segment (start 104.851934 103.34) (end 112.44 103.34) (width 0.75) (layer "F.Cu") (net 8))
 (segment (start 104.4 104.545) (end 104.4 103.791934) (width 0.75) (layer "F.Cu") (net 8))
 (segment (start 113 103.9) (end 113 105) (width 0.75) (layer "F.Cu") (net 8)))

